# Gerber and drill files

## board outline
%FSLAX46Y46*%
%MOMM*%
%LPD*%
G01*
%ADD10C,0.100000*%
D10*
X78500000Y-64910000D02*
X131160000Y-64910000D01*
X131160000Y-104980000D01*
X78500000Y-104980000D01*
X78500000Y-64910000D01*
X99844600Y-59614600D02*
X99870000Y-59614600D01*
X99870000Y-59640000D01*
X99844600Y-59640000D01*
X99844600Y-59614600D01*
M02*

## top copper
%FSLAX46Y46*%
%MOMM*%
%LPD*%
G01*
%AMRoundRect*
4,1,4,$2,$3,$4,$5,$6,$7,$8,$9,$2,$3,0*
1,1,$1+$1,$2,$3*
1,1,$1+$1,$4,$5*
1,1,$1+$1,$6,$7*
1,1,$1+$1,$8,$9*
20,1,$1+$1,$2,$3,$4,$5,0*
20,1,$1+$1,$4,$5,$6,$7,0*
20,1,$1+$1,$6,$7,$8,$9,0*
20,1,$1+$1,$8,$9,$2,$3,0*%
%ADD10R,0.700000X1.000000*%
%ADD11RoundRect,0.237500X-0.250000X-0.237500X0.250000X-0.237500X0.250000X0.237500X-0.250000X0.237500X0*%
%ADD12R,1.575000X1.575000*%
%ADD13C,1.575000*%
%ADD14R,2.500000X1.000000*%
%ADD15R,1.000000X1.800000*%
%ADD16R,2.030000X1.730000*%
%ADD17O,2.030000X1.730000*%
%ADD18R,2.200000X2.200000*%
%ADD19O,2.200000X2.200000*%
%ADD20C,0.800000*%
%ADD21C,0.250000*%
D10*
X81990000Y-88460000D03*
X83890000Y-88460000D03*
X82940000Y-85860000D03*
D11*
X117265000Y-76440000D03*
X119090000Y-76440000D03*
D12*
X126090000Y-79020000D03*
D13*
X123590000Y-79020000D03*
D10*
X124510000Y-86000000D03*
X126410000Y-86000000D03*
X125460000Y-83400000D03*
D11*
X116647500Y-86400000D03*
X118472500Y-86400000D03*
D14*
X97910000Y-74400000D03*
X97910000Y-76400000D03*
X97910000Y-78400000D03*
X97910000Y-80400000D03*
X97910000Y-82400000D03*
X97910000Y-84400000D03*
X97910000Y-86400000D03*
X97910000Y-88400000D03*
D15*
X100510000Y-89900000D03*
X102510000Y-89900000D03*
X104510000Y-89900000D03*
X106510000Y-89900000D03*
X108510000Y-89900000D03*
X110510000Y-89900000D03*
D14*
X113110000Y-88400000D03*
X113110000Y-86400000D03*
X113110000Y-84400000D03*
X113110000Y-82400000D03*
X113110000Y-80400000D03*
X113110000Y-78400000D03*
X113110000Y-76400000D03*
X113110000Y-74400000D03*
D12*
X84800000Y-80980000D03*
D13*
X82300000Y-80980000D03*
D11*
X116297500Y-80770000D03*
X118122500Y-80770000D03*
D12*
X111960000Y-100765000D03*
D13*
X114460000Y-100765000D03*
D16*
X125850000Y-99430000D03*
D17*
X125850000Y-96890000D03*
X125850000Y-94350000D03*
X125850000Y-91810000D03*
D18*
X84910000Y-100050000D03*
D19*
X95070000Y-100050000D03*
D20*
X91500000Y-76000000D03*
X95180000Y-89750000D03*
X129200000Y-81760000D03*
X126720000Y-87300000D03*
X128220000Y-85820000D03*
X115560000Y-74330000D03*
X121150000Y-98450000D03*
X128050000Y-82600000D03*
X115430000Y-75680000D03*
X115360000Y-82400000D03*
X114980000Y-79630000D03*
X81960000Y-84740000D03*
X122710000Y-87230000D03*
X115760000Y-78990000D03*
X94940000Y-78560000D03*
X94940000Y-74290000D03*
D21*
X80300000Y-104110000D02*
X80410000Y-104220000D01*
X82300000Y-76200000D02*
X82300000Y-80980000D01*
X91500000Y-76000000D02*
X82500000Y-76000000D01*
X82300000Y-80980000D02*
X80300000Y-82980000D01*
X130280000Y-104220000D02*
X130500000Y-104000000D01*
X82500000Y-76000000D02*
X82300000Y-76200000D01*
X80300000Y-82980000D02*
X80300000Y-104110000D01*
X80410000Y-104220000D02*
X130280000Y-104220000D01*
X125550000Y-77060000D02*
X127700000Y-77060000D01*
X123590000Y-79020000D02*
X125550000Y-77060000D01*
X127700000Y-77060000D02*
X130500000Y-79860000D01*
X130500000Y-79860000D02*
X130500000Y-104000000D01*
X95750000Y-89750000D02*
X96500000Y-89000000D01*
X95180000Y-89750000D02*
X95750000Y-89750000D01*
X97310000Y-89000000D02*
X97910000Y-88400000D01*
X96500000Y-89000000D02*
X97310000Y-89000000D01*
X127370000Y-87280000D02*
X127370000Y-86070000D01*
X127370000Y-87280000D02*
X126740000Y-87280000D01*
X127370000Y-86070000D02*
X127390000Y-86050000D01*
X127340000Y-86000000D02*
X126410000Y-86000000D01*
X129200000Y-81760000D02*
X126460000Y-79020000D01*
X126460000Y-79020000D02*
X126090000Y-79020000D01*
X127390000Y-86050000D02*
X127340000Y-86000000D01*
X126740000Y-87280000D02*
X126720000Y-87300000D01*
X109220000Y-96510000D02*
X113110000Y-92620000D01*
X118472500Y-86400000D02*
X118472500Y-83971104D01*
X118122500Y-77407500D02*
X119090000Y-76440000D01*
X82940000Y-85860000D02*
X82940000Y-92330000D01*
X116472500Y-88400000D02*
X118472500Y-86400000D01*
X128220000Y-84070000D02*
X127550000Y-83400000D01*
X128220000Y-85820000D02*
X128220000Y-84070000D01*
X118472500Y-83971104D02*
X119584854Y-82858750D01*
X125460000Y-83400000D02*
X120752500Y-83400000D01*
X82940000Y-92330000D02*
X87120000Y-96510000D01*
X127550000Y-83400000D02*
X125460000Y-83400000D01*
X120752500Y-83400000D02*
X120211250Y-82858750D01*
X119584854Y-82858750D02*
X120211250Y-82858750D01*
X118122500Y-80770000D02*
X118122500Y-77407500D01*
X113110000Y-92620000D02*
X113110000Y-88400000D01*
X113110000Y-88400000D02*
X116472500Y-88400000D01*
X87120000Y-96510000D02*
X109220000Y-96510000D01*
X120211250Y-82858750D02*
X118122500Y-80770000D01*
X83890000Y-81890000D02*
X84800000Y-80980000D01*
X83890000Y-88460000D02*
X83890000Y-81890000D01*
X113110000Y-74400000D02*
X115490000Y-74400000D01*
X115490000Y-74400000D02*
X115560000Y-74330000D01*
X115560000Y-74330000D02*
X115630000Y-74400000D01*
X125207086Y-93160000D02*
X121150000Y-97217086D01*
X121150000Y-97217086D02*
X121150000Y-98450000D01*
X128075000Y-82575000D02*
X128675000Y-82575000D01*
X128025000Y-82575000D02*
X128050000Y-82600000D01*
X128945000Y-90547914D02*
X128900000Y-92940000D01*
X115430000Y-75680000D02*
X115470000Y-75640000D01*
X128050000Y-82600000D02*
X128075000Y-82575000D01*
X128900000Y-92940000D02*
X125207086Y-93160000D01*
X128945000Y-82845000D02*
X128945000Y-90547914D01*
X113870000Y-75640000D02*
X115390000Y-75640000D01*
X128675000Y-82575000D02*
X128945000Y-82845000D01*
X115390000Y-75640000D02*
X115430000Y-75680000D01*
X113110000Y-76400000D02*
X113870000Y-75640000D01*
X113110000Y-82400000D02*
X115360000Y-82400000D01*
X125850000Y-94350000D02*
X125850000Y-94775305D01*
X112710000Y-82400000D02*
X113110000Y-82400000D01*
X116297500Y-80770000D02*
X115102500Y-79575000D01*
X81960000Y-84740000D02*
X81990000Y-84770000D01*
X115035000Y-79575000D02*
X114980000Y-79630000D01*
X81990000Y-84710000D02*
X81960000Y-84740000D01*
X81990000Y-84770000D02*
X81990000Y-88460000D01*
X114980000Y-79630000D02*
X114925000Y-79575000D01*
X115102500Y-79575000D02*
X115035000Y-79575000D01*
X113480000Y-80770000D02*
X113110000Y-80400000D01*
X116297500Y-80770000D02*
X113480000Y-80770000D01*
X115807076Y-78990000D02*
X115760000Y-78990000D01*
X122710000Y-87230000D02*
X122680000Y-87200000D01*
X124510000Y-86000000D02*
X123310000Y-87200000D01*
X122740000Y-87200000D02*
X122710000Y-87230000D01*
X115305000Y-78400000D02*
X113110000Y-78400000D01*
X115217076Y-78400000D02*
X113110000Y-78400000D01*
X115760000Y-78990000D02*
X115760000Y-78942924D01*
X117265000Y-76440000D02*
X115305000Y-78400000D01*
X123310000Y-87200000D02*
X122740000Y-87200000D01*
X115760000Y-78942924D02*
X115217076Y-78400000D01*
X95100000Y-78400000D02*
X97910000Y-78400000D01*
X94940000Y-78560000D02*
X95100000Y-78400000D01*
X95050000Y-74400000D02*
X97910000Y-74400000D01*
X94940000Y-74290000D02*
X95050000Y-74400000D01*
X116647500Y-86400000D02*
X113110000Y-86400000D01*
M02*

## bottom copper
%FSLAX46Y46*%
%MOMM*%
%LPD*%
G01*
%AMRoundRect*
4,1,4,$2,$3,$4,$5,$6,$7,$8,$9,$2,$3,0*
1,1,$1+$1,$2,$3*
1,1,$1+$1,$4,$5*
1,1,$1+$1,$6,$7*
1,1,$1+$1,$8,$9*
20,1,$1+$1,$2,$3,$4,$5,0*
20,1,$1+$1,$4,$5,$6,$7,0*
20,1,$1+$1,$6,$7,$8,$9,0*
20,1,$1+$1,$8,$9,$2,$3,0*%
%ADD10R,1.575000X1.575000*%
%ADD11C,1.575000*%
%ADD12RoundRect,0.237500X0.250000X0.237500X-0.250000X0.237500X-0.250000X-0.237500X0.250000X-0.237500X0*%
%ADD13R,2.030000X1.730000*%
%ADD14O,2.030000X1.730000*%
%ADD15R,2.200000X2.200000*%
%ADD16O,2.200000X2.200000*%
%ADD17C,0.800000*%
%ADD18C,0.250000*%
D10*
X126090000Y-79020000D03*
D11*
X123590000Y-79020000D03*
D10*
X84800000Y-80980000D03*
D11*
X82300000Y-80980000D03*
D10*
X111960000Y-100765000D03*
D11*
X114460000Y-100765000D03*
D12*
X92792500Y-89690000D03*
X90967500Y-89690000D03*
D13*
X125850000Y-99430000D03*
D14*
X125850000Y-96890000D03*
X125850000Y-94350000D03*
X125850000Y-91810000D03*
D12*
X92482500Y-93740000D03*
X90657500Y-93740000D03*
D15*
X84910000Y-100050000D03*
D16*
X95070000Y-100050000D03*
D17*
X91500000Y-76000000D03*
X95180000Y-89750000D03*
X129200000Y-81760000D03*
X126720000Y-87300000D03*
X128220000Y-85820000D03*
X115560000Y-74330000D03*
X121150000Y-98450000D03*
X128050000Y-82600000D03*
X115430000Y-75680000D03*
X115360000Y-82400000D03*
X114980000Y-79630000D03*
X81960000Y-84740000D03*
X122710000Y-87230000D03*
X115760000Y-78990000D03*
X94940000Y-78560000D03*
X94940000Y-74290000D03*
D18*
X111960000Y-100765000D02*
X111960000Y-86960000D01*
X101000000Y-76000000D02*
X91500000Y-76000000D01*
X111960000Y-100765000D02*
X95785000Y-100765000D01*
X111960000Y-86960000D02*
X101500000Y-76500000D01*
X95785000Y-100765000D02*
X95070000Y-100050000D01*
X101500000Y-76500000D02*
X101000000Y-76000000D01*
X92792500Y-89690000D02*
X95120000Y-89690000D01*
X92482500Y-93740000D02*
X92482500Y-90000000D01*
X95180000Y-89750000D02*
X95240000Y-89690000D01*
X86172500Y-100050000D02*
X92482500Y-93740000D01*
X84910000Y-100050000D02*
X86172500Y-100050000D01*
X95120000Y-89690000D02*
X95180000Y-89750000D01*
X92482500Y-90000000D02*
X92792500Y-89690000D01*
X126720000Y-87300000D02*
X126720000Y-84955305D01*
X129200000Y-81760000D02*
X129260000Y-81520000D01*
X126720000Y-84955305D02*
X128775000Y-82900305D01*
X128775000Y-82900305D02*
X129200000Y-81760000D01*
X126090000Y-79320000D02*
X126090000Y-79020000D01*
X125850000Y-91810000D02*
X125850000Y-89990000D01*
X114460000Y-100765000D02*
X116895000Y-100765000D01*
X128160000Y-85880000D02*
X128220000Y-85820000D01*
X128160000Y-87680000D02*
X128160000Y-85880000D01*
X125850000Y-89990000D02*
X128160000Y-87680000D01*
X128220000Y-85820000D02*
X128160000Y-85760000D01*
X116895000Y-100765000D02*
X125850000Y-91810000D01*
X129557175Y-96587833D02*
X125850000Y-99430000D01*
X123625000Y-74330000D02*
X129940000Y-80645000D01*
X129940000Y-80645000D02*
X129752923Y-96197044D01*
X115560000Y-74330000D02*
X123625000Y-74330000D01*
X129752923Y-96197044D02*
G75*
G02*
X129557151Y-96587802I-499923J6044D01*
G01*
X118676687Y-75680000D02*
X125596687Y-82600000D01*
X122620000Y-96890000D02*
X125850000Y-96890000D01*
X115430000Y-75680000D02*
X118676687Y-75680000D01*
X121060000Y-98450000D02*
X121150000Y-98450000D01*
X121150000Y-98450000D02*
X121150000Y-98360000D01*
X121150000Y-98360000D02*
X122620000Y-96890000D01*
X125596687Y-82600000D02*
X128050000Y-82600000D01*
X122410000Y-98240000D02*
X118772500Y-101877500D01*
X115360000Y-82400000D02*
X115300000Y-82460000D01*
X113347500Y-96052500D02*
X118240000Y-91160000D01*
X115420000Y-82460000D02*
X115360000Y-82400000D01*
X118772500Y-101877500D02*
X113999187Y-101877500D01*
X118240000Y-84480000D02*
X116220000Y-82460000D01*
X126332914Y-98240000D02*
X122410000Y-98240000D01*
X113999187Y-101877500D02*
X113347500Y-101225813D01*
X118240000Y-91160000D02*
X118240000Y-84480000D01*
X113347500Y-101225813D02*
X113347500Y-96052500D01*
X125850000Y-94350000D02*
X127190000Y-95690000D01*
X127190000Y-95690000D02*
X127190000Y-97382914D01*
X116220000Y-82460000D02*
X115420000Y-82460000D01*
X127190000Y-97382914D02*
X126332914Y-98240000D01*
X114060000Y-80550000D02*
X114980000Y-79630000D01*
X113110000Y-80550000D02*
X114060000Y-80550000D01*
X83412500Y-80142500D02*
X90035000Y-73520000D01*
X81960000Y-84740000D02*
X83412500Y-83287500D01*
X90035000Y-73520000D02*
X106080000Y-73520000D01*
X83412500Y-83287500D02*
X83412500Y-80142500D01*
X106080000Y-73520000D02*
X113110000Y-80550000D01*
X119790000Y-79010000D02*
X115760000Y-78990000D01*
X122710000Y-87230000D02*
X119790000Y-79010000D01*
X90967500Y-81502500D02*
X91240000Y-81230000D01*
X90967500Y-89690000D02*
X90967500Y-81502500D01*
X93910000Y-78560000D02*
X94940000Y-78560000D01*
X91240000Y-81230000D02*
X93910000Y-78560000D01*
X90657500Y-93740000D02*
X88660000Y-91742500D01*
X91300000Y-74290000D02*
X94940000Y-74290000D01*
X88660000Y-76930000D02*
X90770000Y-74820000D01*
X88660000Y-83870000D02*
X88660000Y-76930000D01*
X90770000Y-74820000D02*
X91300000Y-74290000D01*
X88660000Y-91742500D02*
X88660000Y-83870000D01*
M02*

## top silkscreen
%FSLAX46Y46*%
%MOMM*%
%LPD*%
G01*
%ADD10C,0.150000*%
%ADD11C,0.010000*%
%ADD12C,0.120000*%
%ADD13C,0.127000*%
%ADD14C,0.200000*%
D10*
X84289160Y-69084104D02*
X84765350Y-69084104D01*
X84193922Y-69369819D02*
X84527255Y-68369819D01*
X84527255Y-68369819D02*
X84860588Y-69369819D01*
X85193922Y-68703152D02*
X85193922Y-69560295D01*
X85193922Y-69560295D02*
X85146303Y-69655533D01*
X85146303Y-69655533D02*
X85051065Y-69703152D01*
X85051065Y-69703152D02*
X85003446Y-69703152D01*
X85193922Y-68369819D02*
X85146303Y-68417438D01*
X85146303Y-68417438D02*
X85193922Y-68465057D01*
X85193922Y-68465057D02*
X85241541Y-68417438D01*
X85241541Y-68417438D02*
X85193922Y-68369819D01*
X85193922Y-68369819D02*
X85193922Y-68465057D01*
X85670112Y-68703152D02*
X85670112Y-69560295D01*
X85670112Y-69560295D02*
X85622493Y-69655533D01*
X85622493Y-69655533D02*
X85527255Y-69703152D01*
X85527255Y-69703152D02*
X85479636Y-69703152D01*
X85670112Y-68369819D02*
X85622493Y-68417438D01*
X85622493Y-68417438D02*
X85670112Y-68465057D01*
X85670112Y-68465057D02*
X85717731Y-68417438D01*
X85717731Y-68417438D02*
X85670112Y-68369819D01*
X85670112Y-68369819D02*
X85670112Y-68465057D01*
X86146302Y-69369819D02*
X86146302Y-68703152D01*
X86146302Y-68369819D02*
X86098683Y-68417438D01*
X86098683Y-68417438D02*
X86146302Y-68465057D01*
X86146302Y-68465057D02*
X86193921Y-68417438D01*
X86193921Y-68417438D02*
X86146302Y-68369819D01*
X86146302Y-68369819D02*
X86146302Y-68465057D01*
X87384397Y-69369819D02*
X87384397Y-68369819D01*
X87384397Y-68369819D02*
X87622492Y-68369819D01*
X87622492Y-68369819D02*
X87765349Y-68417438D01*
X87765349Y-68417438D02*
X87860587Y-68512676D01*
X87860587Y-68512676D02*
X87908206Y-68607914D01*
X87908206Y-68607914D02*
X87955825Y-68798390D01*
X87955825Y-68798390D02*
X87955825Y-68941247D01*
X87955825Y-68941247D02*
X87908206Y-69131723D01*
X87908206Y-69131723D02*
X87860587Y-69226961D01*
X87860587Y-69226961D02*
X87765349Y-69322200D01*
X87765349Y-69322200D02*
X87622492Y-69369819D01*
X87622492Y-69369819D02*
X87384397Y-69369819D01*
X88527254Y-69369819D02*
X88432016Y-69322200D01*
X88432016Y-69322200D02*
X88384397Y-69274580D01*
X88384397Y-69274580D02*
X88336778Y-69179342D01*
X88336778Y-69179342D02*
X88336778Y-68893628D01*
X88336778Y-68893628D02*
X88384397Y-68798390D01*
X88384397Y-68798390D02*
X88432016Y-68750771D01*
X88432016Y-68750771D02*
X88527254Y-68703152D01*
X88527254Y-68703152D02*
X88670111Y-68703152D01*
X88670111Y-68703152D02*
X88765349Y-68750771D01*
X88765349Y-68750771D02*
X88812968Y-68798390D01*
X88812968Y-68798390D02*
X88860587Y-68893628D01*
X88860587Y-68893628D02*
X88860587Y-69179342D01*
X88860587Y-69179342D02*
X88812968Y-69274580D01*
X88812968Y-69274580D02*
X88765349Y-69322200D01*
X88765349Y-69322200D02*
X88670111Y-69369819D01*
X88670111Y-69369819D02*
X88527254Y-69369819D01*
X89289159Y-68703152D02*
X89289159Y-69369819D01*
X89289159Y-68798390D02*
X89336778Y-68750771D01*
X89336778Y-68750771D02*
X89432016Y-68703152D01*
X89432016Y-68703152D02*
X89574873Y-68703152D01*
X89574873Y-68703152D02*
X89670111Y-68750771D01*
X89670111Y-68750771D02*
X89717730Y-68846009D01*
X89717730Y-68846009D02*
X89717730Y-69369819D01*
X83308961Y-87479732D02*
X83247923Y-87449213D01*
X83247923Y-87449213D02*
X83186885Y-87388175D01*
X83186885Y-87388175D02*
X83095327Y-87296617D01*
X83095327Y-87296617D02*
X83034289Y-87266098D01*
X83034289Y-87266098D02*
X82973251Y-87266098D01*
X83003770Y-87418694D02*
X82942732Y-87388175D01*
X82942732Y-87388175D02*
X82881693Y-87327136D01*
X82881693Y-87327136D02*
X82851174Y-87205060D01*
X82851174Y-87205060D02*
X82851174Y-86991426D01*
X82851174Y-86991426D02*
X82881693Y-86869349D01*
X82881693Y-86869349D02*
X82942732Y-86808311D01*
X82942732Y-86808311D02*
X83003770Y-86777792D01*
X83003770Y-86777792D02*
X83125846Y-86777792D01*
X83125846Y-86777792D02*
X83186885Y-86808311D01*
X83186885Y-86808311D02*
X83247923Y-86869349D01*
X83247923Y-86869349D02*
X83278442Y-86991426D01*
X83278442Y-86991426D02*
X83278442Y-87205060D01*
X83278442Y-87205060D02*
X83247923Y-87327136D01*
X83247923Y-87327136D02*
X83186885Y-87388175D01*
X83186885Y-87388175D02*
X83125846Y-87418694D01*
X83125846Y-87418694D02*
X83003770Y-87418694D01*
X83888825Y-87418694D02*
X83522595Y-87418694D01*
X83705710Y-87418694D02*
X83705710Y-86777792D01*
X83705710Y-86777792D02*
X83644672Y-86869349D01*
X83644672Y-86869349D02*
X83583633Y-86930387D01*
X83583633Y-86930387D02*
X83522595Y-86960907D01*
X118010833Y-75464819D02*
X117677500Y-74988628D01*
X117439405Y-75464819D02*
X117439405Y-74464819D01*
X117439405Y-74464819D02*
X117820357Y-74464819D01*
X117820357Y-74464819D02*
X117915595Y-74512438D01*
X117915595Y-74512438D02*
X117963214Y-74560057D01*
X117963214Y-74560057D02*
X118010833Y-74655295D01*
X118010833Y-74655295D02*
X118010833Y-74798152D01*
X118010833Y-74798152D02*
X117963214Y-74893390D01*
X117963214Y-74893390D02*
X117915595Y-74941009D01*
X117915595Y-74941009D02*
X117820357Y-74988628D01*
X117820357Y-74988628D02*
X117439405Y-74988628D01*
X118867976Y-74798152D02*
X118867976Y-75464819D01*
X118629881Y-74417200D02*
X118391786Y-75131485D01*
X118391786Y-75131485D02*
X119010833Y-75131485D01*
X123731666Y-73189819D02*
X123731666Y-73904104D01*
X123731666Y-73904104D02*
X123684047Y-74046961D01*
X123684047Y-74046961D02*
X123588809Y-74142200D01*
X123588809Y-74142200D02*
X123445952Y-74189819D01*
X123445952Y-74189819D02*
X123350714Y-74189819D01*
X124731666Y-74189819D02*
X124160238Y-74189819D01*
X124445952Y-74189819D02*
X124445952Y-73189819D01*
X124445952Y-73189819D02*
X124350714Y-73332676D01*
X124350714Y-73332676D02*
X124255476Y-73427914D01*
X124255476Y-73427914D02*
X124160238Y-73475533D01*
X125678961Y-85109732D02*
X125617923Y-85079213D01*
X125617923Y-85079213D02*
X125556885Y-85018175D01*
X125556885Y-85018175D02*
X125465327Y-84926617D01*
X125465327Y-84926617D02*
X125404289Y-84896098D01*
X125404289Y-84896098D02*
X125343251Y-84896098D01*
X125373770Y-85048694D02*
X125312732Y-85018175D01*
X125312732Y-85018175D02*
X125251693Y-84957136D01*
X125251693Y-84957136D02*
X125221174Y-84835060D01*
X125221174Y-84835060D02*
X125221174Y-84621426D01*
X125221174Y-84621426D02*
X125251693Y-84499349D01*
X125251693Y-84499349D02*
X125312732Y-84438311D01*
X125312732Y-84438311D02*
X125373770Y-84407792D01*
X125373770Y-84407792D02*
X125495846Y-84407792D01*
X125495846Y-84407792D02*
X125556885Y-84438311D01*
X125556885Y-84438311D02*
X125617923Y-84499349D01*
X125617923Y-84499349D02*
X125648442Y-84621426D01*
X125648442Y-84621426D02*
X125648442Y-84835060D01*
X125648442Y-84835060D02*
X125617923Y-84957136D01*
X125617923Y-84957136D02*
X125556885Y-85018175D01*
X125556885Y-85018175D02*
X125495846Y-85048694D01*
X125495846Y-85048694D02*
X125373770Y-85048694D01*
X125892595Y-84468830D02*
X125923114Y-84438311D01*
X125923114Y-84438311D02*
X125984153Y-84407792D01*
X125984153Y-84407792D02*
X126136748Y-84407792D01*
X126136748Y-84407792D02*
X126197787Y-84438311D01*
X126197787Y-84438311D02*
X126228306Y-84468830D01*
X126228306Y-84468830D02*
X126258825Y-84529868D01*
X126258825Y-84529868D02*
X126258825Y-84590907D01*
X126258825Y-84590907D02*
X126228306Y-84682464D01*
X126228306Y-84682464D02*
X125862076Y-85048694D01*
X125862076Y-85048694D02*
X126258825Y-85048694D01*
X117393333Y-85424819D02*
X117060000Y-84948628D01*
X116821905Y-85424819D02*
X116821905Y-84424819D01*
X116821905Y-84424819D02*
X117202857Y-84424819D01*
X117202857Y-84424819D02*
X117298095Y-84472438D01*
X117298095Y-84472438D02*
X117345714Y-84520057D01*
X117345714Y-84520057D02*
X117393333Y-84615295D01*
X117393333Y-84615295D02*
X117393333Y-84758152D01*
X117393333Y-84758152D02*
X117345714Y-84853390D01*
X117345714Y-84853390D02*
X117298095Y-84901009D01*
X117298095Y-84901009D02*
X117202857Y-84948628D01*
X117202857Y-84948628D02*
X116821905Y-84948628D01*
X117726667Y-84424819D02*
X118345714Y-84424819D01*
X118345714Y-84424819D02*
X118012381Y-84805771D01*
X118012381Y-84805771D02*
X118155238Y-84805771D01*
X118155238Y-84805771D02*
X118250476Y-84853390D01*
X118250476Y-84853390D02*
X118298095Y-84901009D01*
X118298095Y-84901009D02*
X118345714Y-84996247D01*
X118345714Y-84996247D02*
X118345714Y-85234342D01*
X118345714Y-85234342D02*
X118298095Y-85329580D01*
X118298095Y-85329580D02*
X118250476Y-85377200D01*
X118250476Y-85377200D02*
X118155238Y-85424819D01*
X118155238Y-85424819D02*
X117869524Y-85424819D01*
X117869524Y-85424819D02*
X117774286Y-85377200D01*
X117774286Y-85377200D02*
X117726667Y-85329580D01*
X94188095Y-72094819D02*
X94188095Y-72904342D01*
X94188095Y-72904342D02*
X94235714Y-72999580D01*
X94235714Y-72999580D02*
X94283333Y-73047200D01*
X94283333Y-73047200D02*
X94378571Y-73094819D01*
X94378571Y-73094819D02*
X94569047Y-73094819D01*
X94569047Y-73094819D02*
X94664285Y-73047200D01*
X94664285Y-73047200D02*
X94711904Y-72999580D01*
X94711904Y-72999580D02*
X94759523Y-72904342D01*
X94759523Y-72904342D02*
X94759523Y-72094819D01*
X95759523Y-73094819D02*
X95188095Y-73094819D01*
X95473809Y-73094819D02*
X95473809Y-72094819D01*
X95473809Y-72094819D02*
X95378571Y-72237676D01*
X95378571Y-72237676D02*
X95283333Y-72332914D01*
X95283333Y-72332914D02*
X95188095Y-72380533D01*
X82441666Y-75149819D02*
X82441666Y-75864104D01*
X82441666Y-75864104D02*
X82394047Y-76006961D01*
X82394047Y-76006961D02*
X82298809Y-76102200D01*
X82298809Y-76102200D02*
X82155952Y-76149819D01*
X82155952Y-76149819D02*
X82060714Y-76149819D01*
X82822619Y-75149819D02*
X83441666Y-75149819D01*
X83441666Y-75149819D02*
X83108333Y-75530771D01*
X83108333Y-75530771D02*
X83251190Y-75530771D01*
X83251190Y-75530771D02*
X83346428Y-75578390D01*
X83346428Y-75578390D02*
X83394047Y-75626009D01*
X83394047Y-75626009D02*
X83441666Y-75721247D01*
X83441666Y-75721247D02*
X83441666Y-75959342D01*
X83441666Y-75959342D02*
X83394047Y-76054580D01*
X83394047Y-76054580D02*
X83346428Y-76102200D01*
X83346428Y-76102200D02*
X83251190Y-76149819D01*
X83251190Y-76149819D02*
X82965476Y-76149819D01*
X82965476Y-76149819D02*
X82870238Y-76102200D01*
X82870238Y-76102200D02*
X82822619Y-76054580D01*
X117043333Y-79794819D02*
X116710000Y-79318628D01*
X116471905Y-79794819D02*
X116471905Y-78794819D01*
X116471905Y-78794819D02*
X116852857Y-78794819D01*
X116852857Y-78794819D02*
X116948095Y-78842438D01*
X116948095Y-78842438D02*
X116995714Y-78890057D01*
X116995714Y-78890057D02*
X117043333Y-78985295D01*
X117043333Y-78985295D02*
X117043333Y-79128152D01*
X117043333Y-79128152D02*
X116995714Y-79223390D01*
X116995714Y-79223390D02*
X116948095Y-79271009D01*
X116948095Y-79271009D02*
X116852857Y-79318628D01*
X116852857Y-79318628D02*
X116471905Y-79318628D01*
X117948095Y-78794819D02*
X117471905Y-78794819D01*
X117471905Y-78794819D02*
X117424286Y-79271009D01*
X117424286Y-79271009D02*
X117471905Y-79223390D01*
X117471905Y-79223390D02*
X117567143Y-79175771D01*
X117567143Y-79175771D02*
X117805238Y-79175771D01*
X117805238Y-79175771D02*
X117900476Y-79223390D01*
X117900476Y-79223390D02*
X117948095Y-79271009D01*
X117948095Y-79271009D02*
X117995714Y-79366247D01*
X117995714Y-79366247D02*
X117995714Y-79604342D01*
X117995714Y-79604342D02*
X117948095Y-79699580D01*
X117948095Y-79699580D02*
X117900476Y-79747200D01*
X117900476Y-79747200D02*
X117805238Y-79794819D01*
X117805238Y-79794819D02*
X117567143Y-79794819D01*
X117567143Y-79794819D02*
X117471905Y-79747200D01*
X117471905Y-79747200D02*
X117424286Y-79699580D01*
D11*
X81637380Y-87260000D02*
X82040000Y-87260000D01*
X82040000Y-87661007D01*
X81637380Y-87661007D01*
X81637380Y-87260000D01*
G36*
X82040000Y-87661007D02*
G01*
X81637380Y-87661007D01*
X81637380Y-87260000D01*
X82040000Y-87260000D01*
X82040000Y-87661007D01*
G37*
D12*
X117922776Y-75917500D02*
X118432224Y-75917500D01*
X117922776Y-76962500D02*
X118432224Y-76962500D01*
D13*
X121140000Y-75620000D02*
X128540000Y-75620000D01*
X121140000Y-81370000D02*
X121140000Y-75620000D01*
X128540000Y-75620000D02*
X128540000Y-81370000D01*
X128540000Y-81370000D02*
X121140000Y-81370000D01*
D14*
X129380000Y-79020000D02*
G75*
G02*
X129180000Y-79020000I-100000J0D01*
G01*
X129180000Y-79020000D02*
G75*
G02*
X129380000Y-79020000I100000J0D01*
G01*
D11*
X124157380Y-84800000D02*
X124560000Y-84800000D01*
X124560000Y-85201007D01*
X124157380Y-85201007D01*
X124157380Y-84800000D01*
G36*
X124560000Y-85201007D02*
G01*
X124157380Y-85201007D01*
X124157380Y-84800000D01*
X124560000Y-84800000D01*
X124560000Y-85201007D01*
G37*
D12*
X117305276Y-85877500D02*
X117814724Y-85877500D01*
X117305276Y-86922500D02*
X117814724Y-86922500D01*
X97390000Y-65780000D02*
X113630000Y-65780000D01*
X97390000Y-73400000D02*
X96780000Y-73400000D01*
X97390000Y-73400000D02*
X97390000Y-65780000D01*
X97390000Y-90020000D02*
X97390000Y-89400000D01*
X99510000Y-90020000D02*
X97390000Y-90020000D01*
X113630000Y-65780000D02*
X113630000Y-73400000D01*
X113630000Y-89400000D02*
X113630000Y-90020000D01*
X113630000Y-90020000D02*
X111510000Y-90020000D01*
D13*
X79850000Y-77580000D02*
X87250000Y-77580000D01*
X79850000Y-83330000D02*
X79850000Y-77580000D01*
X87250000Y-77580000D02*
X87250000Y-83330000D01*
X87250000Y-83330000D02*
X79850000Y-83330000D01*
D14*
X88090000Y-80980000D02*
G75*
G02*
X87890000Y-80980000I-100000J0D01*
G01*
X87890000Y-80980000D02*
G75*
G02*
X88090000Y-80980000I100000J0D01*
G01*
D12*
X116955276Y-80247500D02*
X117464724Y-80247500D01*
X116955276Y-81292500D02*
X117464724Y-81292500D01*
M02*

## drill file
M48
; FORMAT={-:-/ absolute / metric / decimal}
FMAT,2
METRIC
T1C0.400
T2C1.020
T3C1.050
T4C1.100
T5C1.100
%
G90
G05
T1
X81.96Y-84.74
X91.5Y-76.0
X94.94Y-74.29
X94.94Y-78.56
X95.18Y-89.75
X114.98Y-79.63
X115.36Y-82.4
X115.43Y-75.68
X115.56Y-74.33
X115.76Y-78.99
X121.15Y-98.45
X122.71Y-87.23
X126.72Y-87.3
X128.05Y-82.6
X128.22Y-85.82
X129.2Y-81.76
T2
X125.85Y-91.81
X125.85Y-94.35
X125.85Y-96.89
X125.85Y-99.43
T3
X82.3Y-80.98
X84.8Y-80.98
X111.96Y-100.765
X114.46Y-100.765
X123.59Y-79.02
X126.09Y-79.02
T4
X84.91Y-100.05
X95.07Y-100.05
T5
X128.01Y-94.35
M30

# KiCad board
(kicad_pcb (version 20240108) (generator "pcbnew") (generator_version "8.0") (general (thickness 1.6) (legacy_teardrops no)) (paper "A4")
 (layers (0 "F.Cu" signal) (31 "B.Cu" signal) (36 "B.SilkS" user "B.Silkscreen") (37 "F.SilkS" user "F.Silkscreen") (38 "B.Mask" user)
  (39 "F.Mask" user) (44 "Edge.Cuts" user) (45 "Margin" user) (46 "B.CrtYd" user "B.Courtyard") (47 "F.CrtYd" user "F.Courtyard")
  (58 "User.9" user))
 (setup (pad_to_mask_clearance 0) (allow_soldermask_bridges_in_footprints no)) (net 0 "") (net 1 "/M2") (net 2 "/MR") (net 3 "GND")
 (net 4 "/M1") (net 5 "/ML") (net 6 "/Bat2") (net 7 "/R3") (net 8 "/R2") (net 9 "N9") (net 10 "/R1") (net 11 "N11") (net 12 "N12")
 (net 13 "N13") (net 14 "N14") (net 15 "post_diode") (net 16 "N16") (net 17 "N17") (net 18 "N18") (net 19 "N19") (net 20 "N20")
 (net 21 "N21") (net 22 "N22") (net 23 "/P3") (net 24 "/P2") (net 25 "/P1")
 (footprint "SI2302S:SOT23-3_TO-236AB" (layer "F.Cu") (at 82.94 87.16)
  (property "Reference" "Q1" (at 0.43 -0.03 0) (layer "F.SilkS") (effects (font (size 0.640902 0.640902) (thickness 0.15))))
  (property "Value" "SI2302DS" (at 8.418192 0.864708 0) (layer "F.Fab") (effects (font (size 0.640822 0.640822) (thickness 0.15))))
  (fp_poly
   (pts (xy -1.30262 0.1) (xy -0.9 0.1) (xy -0.9 0.501007) (xy -1.30262 0.501007)) (stroke (width 0.01) (type solid)) (fill solid)
   (layer "F.SilkS"))
  (pad "1" smd rect (at -0.95 1.3) (size 0.7 1) (layers "F.Cu" "F.Paste" "F.Mask") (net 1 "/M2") (solder_mask_margin 0.102))
  (pad "2" smd rect (at 0.95 1.3) (size 0.7 1) (layers "F.Cu" "F.Paste" "F.Mask") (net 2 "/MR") (solder_mask_margin 0.102))
  (pad "3" smd rect (at 0 -1.3) (size 0.7 1) (layers "F.Cu" "F.Paste" "F.Mask") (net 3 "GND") (solder_mask_margin 0.102)))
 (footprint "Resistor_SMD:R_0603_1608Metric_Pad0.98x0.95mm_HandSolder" (layer "F.Cu") (at 118.1775 76.44)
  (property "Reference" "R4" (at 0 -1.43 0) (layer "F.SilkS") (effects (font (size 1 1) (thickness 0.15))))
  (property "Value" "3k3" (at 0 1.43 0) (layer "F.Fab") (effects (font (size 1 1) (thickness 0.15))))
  (fp_line (start -0.254724 -0.5225) (end 0.254724 -0.5225) (stroke (width 0.12) (type solid)) (layer "F.SilkS"))
  (fp_line (start -0.254724 0.5225) (end 0.254724 0.5225) (stroke (width 0.12) (type solid)) (layer "F.SilkS"))
  (pad "1" smd roundrect (at -0.9125 0) (size 0.975 0.95) (layers "F.Cu" "F.Paste" "F.Mask") (roundrect_rratio 0.25) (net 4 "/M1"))
  (pad "2" smd roundrect (at 0.9125 0) (size 0.975 0.95) (layers "F.Cu" "F.Paste" "F.Mask") (roundrect_rratio 0.25) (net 3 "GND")))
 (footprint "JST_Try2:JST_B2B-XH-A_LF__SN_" (layer "F.Cu") (at 124.84 78.495)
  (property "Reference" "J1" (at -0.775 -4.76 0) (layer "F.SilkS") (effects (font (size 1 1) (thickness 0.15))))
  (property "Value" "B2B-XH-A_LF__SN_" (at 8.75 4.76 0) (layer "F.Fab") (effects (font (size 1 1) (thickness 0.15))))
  (fp_line (start -3.7 -2.875) (end 3.7 -2.875) (stroke (width 0.127) (type solid)) (layer "F.SilkS"))
  (fp_line (start -3.7 2.875) (end -3.7 -2.875) (stroke (width 0.127) (type solid)) (layer "F.SilkS"))
  (fp_line (start 3.7 -2.875) (end 3.7 2.875) (stroke (width 0.127) (type solid)) (layer "F.SilkS"))
  (fp_line (start 3.7 2.875) (end -3.7 2.875) (stroke (width 0.127) (type solid)) (layer "F.SilkS"))
  (fp_circle (center 4.44 0.525) (end 4.54 0.525) (stroke (width 0.2) (type solid)) (fill none) (layer "F.SilkS"))
  (pad "1" thru_hole rect (at 1.25 0.525) (size 1.575 1.575) (drill 1.05) (layers "*.Cu" "*.Mask") (remove_unused_layers no) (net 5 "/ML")
   (solder_mask_margin 0.102))
  (pad "2" thru_hole circle (at -1.25 0.525) (size 1.575 1.575) (drill 1.05) (layers "*.Cu" "*.Mask") (remove_unused_layers no)
   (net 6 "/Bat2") (solder_mask_margin 0.102)))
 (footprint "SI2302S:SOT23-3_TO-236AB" (layer "F.Cu") (at 125.46 84.7)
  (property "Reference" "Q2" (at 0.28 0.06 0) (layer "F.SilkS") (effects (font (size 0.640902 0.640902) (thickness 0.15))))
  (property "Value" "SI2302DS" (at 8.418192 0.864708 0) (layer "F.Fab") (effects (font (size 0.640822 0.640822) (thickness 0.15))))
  (fp_poly
   (pts (xy -1.30262 0.1) (xy -0.9 0.1) (xy -0.9 0.501007) (xy -1.30262 0.501007)) (stroke (width 0.01) (type solid)) (fill solid)
   (layer "F.SilkS"))
  (pad "1" smd rect (at -0.95 1.3) (size 0.7 1) (layers "F.Cu" "F.Paste" "F.Mask") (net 4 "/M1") (solder_mask_margin 0.102))
  (pad "2" smd rect (at 0.95 1.3) (size 0.7 1) (layers "F.Cu" "F.Paste" "F.Mask") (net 5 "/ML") (solder_mask_margin 0.102))
  (pad "3" smd rect (at 0 -1.3) (size 0.7 1) (layers "F.Cu" "F.Paste" "F.Mask") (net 3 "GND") (solder_mask_margin 0.102)))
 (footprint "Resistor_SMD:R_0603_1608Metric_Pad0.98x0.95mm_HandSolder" (layer "F.Cu") (at 117.56 86.4)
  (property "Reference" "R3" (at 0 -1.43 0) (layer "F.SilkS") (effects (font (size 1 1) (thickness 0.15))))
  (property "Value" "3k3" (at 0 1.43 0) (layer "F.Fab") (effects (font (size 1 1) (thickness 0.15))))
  (fp_line (start -0.254724 -0.5225) (end 0.254724 -0.5225) (stroke (width 0.12) (type solid)) (layer "F.SilkS"))
  (fp_line (start -0.254724 0.5225) (end 0.254724 0.5225) (stroke (width 0.12) (type solid)) (layer "F.SilkS"))
  (pad "1" smd roundrect (at -0.9125 0) (size 0.975 0.95) (layers "F.Cu" "F.Paste" "F.Mask") (roundrect_rratio 0.25) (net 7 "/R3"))
  (pad "2" smd roundrect (at 0.9125 0) (size 0.975 0.95) (layers "F.Cu" "F.Paste" "F.Mask") (roundrect_rratio 0.25) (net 3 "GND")))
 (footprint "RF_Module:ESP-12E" (layer "F.Cu") (at 105.51 77.9)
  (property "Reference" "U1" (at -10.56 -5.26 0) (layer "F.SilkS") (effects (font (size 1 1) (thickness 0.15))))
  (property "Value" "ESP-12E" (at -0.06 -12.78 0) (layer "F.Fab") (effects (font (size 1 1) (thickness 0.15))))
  (fp_line (start -8.12 -12.12) (end 8.12 -12.12) (stroke (width 0.12) (type solid)) (layer "F.SilkS"))
  (fp_line (start -8.12 -4.5) (end -8.73 -4.5) (stroke (width 0.12) (type solid)) (layer "F.SilkS"))
  (fp_line (start -8.12 -4.5) (end -8.12 -12.12) (stroke (width 0.12) (type solid)) (layer "F.SilkS"))
  (fp_line (start -8.12 12.12) (end -8.12 11.5) (stroke (width 0.12) (type solid)) (layer "F.SilkS"))
  (fp_line (start -6 12.12) (end -8.12 12.12) (stroke (width 0.12) (type solid)) (layer "F.SilkS"))
  (fp_line (start 8.12 -12.12) (end 8.12 -4.5) (stroke (width 0.12) (type solid)) (layer "F.SilkS"))
  (fp_line (start 8.12 11.5) (end 8.12 12.12) (stroke (width 0.12) (type solid)) (layer "F.SilkS"))
  (fp_line (start 8.12 12.12) (end 6 12.12) (stroke (width 0.12) (type solid)) (layer "F.SilkS"))
  (pad "1" smd rect (at -7.6 -3.5) (size 2.5 1) (layers "F.Cu" "F.Mask") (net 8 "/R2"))
  (pad "2" smd rect (at -7.6 -1.5) (size 2.5 1) (layers "F.Cu" "F.Mask") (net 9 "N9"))
  (pad "3" smd rect (at -7.6 0.5) (size 2.5 1) (layers "F.Cu" "F.Mask") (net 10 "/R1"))
  (pad "4" smd rect (at -7.6 2.5) (size 2.5 1) (layers "F.Cu" "F.Mask") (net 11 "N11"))
  (pad "5" smd rect (at -7.6 4.5) (size 2.5 1) (layers "F.Cu" "F.Mask") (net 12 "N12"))
  (pad "6" smd rect (at -7.6 6.5) (size 2.5 1) (layers "F.Cu" "F.Mask") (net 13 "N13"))
  (pad "7" smd rect (at -7.6 8.5) (size 2.5 1) (layers "F.Cu" "F.Mask") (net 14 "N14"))
  (pad "8" smd rect (at -7.6 10.5) (size 2.5 1) (layers "F.Cu" "F.Mask") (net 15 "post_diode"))
  (pad "9" smd rect (at -5 12) (size 1 1.8) (layers "F.Cu" "F.Mask") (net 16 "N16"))
  (pad "10" smd rect (at -3 12) (size 1 1.8) (layers "F.Cu" "F.Mask") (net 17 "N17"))
  (pad "11" smd rect (at -1 12) (size 1 1.8) (layers "F.Cu" "F.Mask") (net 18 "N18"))
  (pad "12" smd rect (at 1 12) (size 1 1.8) (layers "F.Cu" "F.Mask") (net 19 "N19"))
  (pad "13" smd rect (at 3 12) (size 1 1.8) (layers "F.Cu" "F.Mask") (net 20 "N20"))
  (pad "14" smd rect (at 5 12) (size 1 1.8) (layers "F.Cu" "F.Mask") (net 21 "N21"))
  (pad "15" smd rect (at 7.6 10.5) (size 2.5 1) (layers "F.Cu" "F.Mask") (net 3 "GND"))
  (pad "16" smd rect (at 7.6 8.5) (size 2.5 1) (layers "F.Cu" "F.Mask") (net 7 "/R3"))
  (pad "17" smd rect (at 7.6 6.5) (size 2.5 1) (layers "F.Cu" "F.Mask") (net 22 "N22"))
  (pad "18" smd rect (at 7.6 4.5) (size 2.5 1) (layers "F.Cu" "F.Mask") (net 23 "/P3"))
  (pad "19" smd rect (at 7.6 2.5) (size 2.5 1) (layers "F.Cu" "F.Mask") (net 1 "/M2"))
  (pad "20" smd rect (at 7.6 0.5) (size 2.5 1) (layers "F.Cu" "F.Mask") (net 4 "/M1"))
  (pad "21" smd rect (at 7.6 -1.5) (size 2.5 1) (layers "F.Cu" "F.Mask") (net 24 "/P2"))
  (pad "22" smd rect (at 7.6 -3.5) (size 2.5 1) (layers "F.Cu" "F.Mask") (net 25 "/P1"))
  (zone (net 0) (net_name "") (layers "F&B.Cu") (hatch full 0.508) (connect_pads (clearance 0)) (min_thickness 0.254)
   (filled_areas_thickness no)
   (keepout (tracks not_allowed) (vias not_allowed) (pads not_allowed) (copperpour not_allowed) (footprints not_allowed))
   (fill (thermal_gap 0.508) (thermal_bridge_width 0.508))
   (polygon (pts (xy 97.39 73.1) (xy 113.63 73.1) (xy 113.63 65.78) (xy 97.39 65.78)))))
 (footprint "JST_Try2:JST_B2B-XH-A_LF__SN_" (layer "F.Cu") (at 83.55 80.455)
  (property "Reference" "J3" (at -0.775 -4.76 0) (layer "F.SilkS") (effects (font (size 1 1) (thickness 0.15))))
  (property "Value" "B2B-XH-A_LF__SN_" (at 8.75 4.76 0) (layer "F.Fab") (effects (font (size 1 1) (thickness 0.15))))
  (fp_line (start -3.7 -2.875) (end 3.7 -2.875) (stroke (width 0.127) (type solid)) (layer "F.SilkS"))
  (fp_line (start -3.7 2.875) (end -3.7 -2.875) (stroke (width 0.127) (type solid)) (layer "F.SilkS"))
  (fp_line (start 3.7 -2.875) (end 3.7 2.875) (stroke (width 0.127) (type solid)) (layer "F.SilkS"))
  (fp_line (start 3.7 2.875) (end -3.7 2.875) (stroke (width 0.127) (type solid)) (layer "F.SilkS"))
  (fp_circle (center 4.44 0.525) (end 4.54 0.525) (stroke (width 0.2) (type solid)) (fill none) (layer "F.SilkS"))
  (pad "1" thru_hole rect (at 1.25 0.525) (size 1.575 1.575) (drill 1.05) (layers "*.Cu" "*.Mask") (remove_unused_layers no) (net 2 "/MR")
   (solder_mask_margin 0.102))
  (pad "2" thru_hole circle (at -1.25 0.525) (size 1.575 1.575) (drill 1.05) (layers "*.Cu" "*.Mask") (remove_unused_layers no)
   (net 6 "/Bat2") (solder_mask_margin 0.102)))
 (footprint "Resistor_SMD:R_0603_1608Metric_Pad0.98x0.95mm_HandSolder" (layer "F.Cu") (at 117.21 80.77)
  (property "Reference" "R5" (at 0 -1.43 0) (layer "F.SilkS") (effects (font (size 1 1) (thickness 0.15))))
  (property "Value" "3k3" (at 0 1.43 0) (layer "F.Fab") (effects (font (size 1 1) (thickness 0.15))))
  (fp_line (start -0.254724 -0.5225) (end 0.254724 -0.5225) (stroke (width 0.12) (type solid)) (layer "F.SilkS"))
  (fp_line (start -0.254724 0.5225) (end 0.254724 0.5225) (stroke (width 0.12) (type solid)) (layer "F.SilkS"))
  (pad "1" smd roundrect (at -0.9125 0) (size 0.975 0.95) (layers "F.Cu" "F.Paste" "F.Mask") (roundrect_rratio 0.25) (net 1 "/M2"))
  (pad "2" smd roundrect (at 0.9125 0) (size 0.975 0.95) (layers "F.Cu" "F.Paste" "F.Mask") (roundrect_rratio 0.25) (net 3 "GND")))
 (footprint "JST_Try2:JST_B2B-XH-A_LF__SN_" (layer "B.Cu") (at 113.21 100.24 180)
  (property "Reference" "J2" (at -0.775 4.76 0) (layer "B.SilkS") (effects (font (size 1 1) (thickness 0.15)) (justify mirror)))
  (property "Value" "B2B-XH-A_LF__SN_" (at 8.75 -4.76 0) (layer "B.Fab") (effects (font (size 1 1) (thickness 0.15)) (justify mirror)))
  (pad "1" thru_hole rect (at 1.25 -0.525 180) (size 1.575 1.575) (drill 1.05) (layers "*.Cu" "*.Mask") (remove_unused_layers no)
   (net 6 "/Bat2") (solder_mask_margin 0.102))
  (pad "2" thru_hole circle (at -1.25 -0.525 180) (size 1.575 1.575) (drill 1.05) (layers "*.Cu" "*.Mask") (remove_unused_layers no)
   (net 3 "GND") (solder_mask_margin 0.102)))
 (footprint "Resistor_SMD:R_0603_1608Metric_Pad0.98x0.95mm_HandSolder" (layer "B.Cu") (at 91.88 89.69 180)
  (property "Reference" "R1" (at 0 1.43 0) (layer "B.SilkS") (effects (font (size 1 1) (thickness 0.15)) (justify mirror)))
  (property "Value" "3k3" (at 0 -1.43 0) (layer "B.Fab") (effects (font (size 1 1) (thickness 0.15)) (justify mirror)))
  (pad "1" smd roundrect (at -0.9125 0 180) (size 0.975 0.95) (layers "B.Cu" "B.Paste" "B.Mask") (roundrect_rratio 0.25)
   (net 15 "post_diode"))
  (pad "2" smd roundrect (at 0.9125 0 180) (size 0.975 0.95) (layers "B.Cu" "B.Paste" "B.Mask") (roundrect_rratio 0.25) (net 10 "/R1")))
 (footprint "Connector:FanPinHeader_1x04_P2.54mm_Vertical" (layer "B.Cu") (at 125.85 99.43 90)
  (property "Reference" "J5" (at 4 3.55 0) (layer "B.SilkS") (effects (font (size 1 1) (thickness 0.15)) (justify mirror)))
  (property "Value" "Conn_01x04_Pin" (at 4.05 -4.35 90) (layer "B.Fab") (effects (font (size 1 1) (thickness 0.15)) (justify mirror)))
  (pad "" np_thru_hole circle (at 5.08 2.16) (size 1.1 1.1) (drill 1.1) (layers "*.Cu" "*.Mask"))
  (pad "1" thru_hole rect (at 0 0) (size 2.03 1.73) (drill 1.02) (layers "*.Cu" "*.Mask") (remove_unused_layers no) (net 25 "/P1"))
  (pad "2" thru_hole oval (at 2.54 0) (size 2.03 1.73) (drill 1.02) (layers "*.Cu" "*.Mask") (remove_unused_layers no) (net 24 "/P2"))
  (pad "3" thru_hole oval (at 5.08 0) (size 2.03 1.73) (drill 1.02) (layers "*.Cu" "*.Mask") (remove_unused_layers no) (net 23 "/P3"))
  (pad "4" thru_hole oval (at 7.62 0) (size 2.03 1.73) (drill 1.02) (layers "*.Cu" "*.Mask") (remove_unused_layers no) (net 3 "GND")))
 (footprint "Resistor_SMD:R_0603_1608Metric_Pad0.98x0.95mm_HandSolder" (layer "B.Cu") (at 91.57 93.74 180)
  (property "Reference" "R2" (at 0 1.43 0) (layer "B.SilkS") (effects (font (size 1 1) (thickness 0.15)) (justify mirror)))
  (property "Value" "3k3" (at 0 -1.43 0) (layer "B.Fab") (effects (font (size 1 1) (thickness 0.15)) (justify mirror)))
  (pad "1" smd roundrect (at -0.9125 0 180) (size 0.975 0.95) (layers "B.Cu" "B.Paste" "B.Mask") (roundrect_rratio 0.25)
   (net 15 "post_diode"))
  (pad "2" smd roundrect (at 0.9125 0 180) (size 0.975 0.95) (layers "B.Cu" "B.Paste" "B.Mask") (roundrect_rratio 0.25) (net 8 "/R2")))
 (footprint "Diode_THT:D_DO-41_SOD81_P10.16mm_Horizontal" (layer "B.Cu") (at 84.91 100.05)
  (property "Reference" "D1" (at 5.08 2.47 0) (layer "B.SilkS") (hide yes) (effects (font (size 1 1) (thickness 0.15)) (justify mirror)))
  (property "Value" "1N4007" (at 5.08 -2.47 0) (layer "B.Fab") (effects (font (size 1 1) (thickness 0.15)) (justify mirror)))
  (pad "1" thru_hole rect (at 0 0) (size 2.2 2.2) (drill 1.1) (layers "*.Cu" "*.Mask") (remove_unused_layers no) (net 15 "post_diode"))
  (pad "2" thru_hole oval (at 10.16 0) (size 2.2 2.2) (drill 1.1) (layers "*.Cu" "*.Mask") (remove_unused_layers no) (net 6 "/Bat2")))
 (gr_rect (start 78.5 64.91) (end 131.16 104.98) (stroke (width 0.1) (type default)) (fill none) (layer "Edge.Cuts"))
 (gr_rect (start 99.8446 59.6146) (end 99.87 59.64) (stroke (width 0.1) (type default)) (fill none) (layer "Edge.Cuts"))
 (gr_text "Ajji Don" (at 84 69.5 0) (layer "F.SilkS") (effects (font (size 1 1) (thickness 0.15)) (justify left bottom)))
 (segment (start 80.3 104.11) (end 80.41 104.22) (width 0.25) (layer "F.Cu") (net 6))
 (segment (start 82.3 76.2) (end 82.3 80.98) (width 0.25) (layer "F.Cu") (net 6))
 (segment (start 91.5 76) (end 82.5 76) (width 0.25) (layer "F.Cu") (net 6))
 (segment (start 82.3 80.98) (end 80.3 82.98) (width 0.25) (layer "F.Cu") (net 6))
 (segment (start 130.28 104.22) (end 130.5 104) (width 0.25) (layer "F.Cu") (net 6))
 (segment (start 82.5 76) (end 82.3 76.2) (width 0.25) (layer "F.Cu") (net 6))
 (segment (start 80.3 82.98) (end 80.3 104.11) (width 0.25) (layer "F.Cu") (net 6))
 (segment (start 80.41 104.22) (end 130.28 104.22) (width 0.25) (layer "F.Cu") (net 6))
 (segment (start 125.55 77.06) (end 127.7 77.06) (width 0.25) (layer "F.Cu") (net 6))
 (segment (start 123.59 79.02) (end 125.55 77.06) (width 0.25) (layer "F.Cu") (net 6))
 (segment (start 127.7 77.06) (end 130.5 79.86) (width 0.25) (layer "F.Cu") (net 6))
 (segment (start 130.5 79.86) (end 130.5 104) (width 0.25) (layer "F.Cu") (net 6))
 (via (at 91.5 76) (size 0.8) (drill 0.4) (layers "F.Cu" "B.Cu") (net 6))
 (segment (start 111.96 100.765) (end 111.96 86.96) (width 0.25) (layer "B.Cu") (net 6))
 (segment (start 101 76) (end 91.5 76) (width 0.25) (layer "B.Cu") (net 6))
 (segment (start 111.96 100.765) (end 95.785 100.765) (width 0.25) (layer "B.Cu") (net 6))
 (segment (start 111.96 86.96) (end 101.5 76.5) (width 0.25) (layer "B.Cu") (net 6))
 (segment (start 95.785 100.765) (end 95.07 100.05) (width 0.25) (layer "B.Cu") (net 6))
 (segment (start 101.5 76.5) (end 101 76) (width 0.25) (layer "B.Cu") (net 6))
 (segment (start 95.75 89.75) (end 96.5 89) (width 0.25) (layer "F.Cu") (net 15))
 (segment (start 95.18 89.75) (end 95.75 89.75) (width 0.25) (layer "F.Cu") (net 15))
 (segment (start 97.31 89) (end 97.91 88.4) (width 0.25) (layer "F.Cu") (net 15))
 (segment (start 96.5 89) (end 97.31 89) (width 0.25) (layer "F.Cu") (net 15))
 (via (at 95.18 89.75) (size 0.8) (drill 0.4) (layers "F.Cu" "B.Cu") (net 15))
 (segment (start 92.7925 89.69) (end 95.12 89.69) (width 0.25) (layer "B.Cu") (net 15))
 (segment (start 92.4825 93.74) (end 92.4825 90) (width 0.25) (layer "B.Cu") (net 15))
 (segment (start 95.18 89.75) (end 95.24 89.69) (width 0.25) (layer "B.Cu") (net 15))
 (segment (start 86.1725 100.05) (end 92.4825 93.74) (width 0.25) (layer "B.Cu") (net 15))
 (segment (start 84.91 100.05) (end 86.1725 100.05) (width 0.25) (layer "B.Cu") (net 15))
 (segment (start 95.12 89.69) (end 95.18 89.75) (width 0.25) (layer "B.Cu") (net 15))
 (segment (start 92.4825 90) (end 92.7925 89.69) (width 0.25) (layer "B.Cu") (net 15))
 (segment (start 127.37 87.28) (end 127.37 86.07) (width 0.25) (layer "F.Cu") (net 5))
 (segment (start 127.37 87.28) (end 126.74 87.28) (width 0.25) (layer "F.Cu") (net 5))
 (segment (start 127.37 86.07) (end 127.39 86.05) (width 0.25) (layer "F.Cu") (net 5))
 (segment (start 127.34 86) (end 126.41 86) (width 0.25) (layer "F.Cu") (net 5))
 (segment (start 129.2 81.76) (end 126.46 79.02) (width 0.25) (layer "F.Cu") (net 5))
 (segment (start 126.46 79.02) (end 126.09 79.02) (width 0.25) (layer "F.Cu") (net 5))
 (segment (start 127.39 86.05) (end 127.34 86) (width 0.25) (layer "F.Cu") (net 5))
 (segment (start 126.74 87.28) (end 126.72 87.3) (width 0.25) (layer "F.Cu") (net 5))
 (via (at 129.2 81.76) (size 0.8) (drill 0.4) (layers "F.Cu" "B.Cu") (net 5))
 (via (at 126.72 87.3) (size 0.8) (drill 0.4) (layers "F.Cu" "B.Cu") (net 5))
 (segment (start 126.72 87.3) (end 126.72 84.955305) (width 0.25) (layer "B.Cu") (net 5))
 (segment (start 129.2 81.76) (end 129.26 81.52) (width 0.25) (layer "B.Cu") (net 5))
 (segment (start 126.72 84.955305) (end 128.775 82.900305) (width 0.25) (layer "B.Cu") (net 5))
 (segment (start 128.775 82.900305) (end 129.2 81.76) (width 0.25) (layer "B.Cu") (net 5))
 (segment (start 126.09 79.32) (end 126.09 79.02) (width 0.25) (layer "B.Cu") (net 5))
 (segment (start 109.22 96.51) (end 113.11 92.62) (width 0.25) (layer "F.Cu") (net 3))
 (segment (start 118.4725 86.4) (end 118.4725 83.971104) (width 0.25) (layer "F.Cu") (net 3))
 (segment (start 118.1225 77.4075) (end 119.09 76.44) (width 0.25) (layer "F.Cu") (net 3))
 (segment (start 82.94 85.86) (end 82.94 92.33) (width 0.25) (layer "F.Cu") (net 3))
 (segment (start 116.4725 88.4) (end 118.4725 86.4) (width 0.25) (layer "F.Cu") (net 3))
 (segment (start 128.22 84.07) (end 127.55 83.4) (width 0.25) (layer "F.Cu") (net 3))
 (segment (start 128.22 85.82) (end 128.22 84.07) (width 0.25) (layer "F.Cu") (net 3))
 (segment (start 118.4725 83.971104) (end 119.584854 82.85875) (width 0.25) (layer "F.Cu") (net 3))
 (segment (start 125.46 83.4) (end 120.7525 83.4) (width 0.25) (layer "F.Cu") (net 3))
 (segment (start 82.94 92.33) (end 87.12 96.51) (width 0.25) (layer "F.Cu") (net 3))
 (segment (start 127.55 83.4) (end 125.46 83.4) (width 0.25) (layer "F.Cu") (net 3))
 (segment (start 120.7525 83.4) (end 120.21125 82.85875) (width 0.25) (layer "F.Cu") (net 3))
 (segment (start 119.584854 82.85875) (end 120.21125 82.85875) (width 0.25) (layer "F.Cu") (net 3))
 (segment (start 118.1225 80.77) (end 118.1225 77.4075) (width 0.25) (layer "F.Cu") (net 3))
 (segment (start 113.11 92.62) (end 113.11 88.4) (width 0.25) (layer "F.Cu") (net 3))
 (segment (start 113.11 88.4) (end 116.4725 88.4) (width 0.25) (layer "F.Cu") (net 3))
 (segment (start 87.12 96.51) (end 109.22 96.51) (width 0.25) (layer "F.Cu") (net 3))
 (segment (start 120.21125 82.85875) (end 118.1225 80.77) (width 0.25) (layer "F.Cu") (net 3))
 (via (at 128.22 85.82) (size 0.8) (drill 0.4) (layers "F.Cu" "B.Cu") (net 3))
 (segment (start 125.85 91.81) (end 125.85 89.99) (width 0.25) (layer "B.Cu") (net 3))
 (segment (start 114.46 100.765) (end 116.895 100.765) (width 0.25) (layer "B.Cu") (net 3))
 (segment (start 128.16 85.88) (end 128.22 85.82) (width 0.25) (layer "B.Cu") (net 3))
 (segment (start 128.16 87.68) (end 128.16 85.88) (width 0.25) (layer "B.Cu") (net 3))
 (segment (start 125.85 89.99) (end 128.16 87.68) (width 0.25) (layer "B.Cu") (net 3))
 (segment (start 128.22 85.82) (end 128.16 85.76) (width 0.25) (layer "B.Cu") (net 3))
 (segment (start 116.895 100.765) (end 125.85 91.81) (width 0.25) (layer "B.Cu") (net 3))
 (segment (start 83.89 81.89) (end 84.8 80.98) (width 0.25) (layer "F.Cu") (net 2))
 (segment (start 83.89 88.46) (end 83.89 81.89) (width 0.25) (layer "F.Cu") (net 2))
 (segment (start 113.11 74.4) (end 115.49 74.4) (width 0.25) (layer "F.Cu") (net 25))
 (segment (start 115.49 74.4) (end 115.56 74.33) (width 0.25) (layer "F.Cu") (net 25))
 (segment (start 115.56 74.33) (end 115.63 74.4) (width 0.25) (layer "F.Cu") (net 25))
 (via (at 115.56 74.33) (size 0.8) (drill 0.4) (layers "F.Cu" "B.Cu") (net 25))
 (segment (start 129.557175 96.587833) (end 125.85 99.43) (width 0.25) (layer "B.Cu") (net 25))
 (segment (start 123.625 74.33) (end 129.94 80.645) (width 0.25) (layer "B.Cu") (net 25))
 (segment (start 129.94 80.645) (end 129.752923 96.197044) (width 0.25) (layer "B.Cu") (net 25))
 (segment (start 115.56 74.33) (end 123.625 74.33) (width 0.25) (layer "B.Cu") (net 25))
 (arc (start 129.752923 96.197044) (mid 129.700011 96.41496) (end 129.557175 96.587833) (width 0.25) (layer "B.Cu") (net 25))
 (segment (start 125.207086 93.16) (end 121.15 97.217086) (width 0.25) (layer "F.Cu") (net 24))
 (segment (start 121.15 97.217086) (end 121.15 98.45) (width 0.25) (layer "F.Cu") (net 24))
 (segment (start 128.075 82.575) (end 128.675 82.575) (width 0.25) (layer "F.Cu") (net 24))
 (segment (start 128.025 82.575) (end 128.05 82.6) (width 0.25) (layer "F.Cu") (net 24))
 (segment (start 128.945 90.547914) (end 128.9 92.94) (width 0.25) (layer "F.Cu") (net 24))
 (segment (start 115.43 75.68) (end 115.47 75.64) (width 0.25) (layer "F.Cu") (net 24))
 (segment (start 128.05 82.6) (end 128.075 82.575) (width 0.25) (layer "F.Cu") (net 24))
 (segment (start 128.9 92.94) (end 125.207086 93.16) (width 0.25) (layer "F.Cu") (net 24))
 (segment (start 128.945 82.845) (end 128.945 90.547914) (width 0.25) (layer "F.Cu") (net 24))
 (segment (start 113.87 75.64) (end 115.39 75.64) (width 0.25) (layer "F.Cu") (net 24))
 (segment (start 128.675 82.575) (end 128.945 82.845) (width 0.25) (layer "F.Cu") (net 24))
 (segment (start 115.39 75.64) (end 115.43 75.68) (width 0.25) (layer "F.Cu") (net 24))
 (segment (start 113.11 76.4) (end 113.87 75.64) (width 0.25) (layer "F.Cu") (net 24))
 (via (at 121.15 98.45) (size 0.8) (drill 0.4) (layers "F.Cu" "B.Cu") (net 24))
 (via (at 128.05 82.6) (size 0.8) (drill 0.4) (layers "F.Cu" "B.Cu") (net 24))
 (via (at 115.43 75.68) (size 0.8) (drill 0.4) (layers "F.Cu" "B.Cu") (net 24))
 (segment (start 118.676687 75.68) (end 125.596687 82.6) (width 0.25) (layer "B.Cu") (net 24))
 (segment (start 122.62 96.89) (end 125.85 96.89) (width 0.25) (layer "B.Cu") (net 24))
 (segment (start 115.43 75.68) (end 118.676687 75.68) (width 0.25) (layer "B.Cu") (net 24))
 (segment (start 121.06 98.45) (end 121.15 98.45) (width 0.25) (layer "B.Cu") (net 24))
 (segment (start 121.15 98.45) (end 121.15 98.36) (width 0.25) (layer "B.Cu") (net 24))
 (segment (start 121.15 98.36) (end 122.62 96.89) (width 0.25) (layer "B.Cu") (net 24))
 (segment (start 125.596687 82.6) (end 128.05 82.6) (width 0.25) (layer "B.Cu") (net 24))
 (segment (start 113.11 82.4) (end 115.36 82.4) (width 0.25) (layer "F.Cu") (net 23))
 (segment (start 125.85 94.35) (end 125.85 94.775305) (width 0.25) (layer "F.Cu") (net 23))
 (segment (start 112.71 82.4) (end 113.11 82.4) (width 0.25) (layer "F.Cu") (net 23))
 (via (at 115.36 82.4) (size 0.8) (drill 0.4) (layers "F.Cu" "B.Cu") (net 23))
 (segment (start 122.41 98.24) (end 118.7725 101.8775) (width 0.25) (layer "B.Cu") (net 23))
 (segment (start 115.36 82.4) (end 115.3 82.46) (width 0.25) (layer "B.Cu") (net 23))
 (segment (start 113.3475 96.0525) (end 118.24 91.16) (width 0.25) (layer "B.Cu") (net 23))
 (segment (start 115.42 82.46) (end 115.36 82.4) (width 0.25) (layer "B.Cu") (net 23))
 (segment (start 118.7725 101.8775) (end 113.999187 101.8775) (width 0.25) (layer "B.Cu") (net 23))
 (segment (start 118.24 84.48) (end 116.22 82.46) (width 0.25) (layer "B.Cu") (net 23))
 (segment (start 126.332914 98.24) (end 122.41 98.24) (width 0.25) (layer "B.Cu") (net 23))
 (segment (start 113.999187 101.8775) (end 113.3475 101.225813) (width 0.25) (layer "B.Cu") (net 23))
 (segment (start 118.24 91.16) (end 118.24 84.48) (width 0.25) (layer "B.Cu") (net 23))
 (segment (start 113.3475 101.225813) (end 113.3475 96.0525) (width 0.25) (layer "B.Cu") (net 23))
 (segment (start 125.85 94.35) (end 127.19 95.69) (width 0.25) (layer "B.Cu") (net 23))
 (segment (start 127.19 95.69) (end 127.19 97.382914) (width 0.25) (layer "B.Cu") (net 23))
 (segment (start 116.22 82.46) (end 115.42 82.46) (width 0.25) (layer "B.Cu") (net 23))
 (segment (start 127.19 97.382914) (end 126.332914 98.24) (width 0.25) (layer "B.Cu") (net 23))
 (segment (start 116.2975 80.77) (end 115.1025 79.575) (width 0.25) (layer "F.Cu") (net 1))
 (segment (start 81.96 84.74) (end 81.99 84.77) (width 0.25) (layer "F.Cu") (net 1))
 (segment (start 115.035 79.575) (end 114.98 79.63) (width 0.25) (layer "F.Cu") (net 1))
 (segment (start 81.99 84.71) (end 81.96 84.74) (width 0.25) (layer "F.Cu") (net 1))
 (segment (start 81.99 84.77) (end 81.99 88.46) (width 0.25) (layer "F.Cu") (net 1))
 (segment (start 114.98 79.63) (end 114.925 79.575) (width 0.25) (layer "F.Cu") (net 1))
 (segment (start 115.1025 79.575) (end 115.035 79.575) (width 0.25) (layer "F.Cu") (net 1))
 (segment (start 113.48 80.77) (end 113.11 80.4) (width 0.25) (layer "F.Cu") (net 1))
 (segment (start 116.2975 80.77) (end 113.48 80.77) (width 0.25) (layer "F.Cu") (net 1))
 (via (at 114.98 79.63) (size 0.8) (drill 0.4) (layers "F.Cu" "B.Cu") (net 1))
 (via (at 81.96 84.74) (size 0.8) (drill 0.4) (layers "F.Cu" "B.Cu") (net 1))
 (segment (start 114.06 80.55) (end 114.98 79.63) (width 0.25) (layer "B.Cu") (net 1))
 (segment (start 113.11 80.55) (end 114.06 80.55) (width 0.25) (layer "B.Cu") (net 1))
 (segment (start 83.4125 80.1425) (end 90.035 73.52) (width 0.25) (layer "B.Cu") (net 1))
 (segment (start 81.96 84.74) (end 83.4125 83.2875) (width 0.25) (layer "B.Cu") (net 1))
 (segment (start 90.035 73.52) (end 106.08 73.52) (width 0.25) (layer "B.Cu") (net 1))
 (segment (start 83.4125 83.2875) (end 83.4125 80.1425) (width 0.25) (layer "B.Cu") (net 1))
 (segment (start 106.08 73.52) (end 113.11 80.55) (width 0.25) (layer "B.Cu") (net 1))
 (segment (start 115.807076 78.99) (end 115.76 78.99) (width 0.25) (layer "F.Cu") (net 4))
 (segment (start 122.71 87.23) (end 122.68 87.2) (width 0.25) (layer "F.Cu") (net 4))
 (segment (start 124.51 86) (end 123.31 87.2) (width 0.25) (layer "F.Cu") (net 4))
 (segment (start 122.74 87.2) (end 122.71 87.23) (width 0.25) (layer "F.Cu") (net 4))
 (segment (start 115.305 78.4) (end 113.11 78.4) (width 0.25) (layer "F.Cu") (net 4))
 (segment (start 115.217076 78.4) (end 113.11 78.4) (width 0.25) (layer "F.Cu") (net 4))
 (segment (start 115.76 78.99) (end 115.76 78.942924) (width 0.25) (layer "F.Cu") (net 4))
 (segment (start 117.265 76.44) (end 115.305 78.4) (width 0.25) (layer "F.Cu") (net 4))
 (segment (start 123.31 87.2) (end 122.74 87.2) (width 0.25) (layer "F.Cu") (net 4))
 (segment (start 115.76 78.942924) (end 115.217076 78.4) (width 0.25) (layer "F.Cu") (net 4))
 (via (at 122.71 87.23) (size 0.8) (drill 0.4) (layers "F.Cu" "B.Cu") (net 4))
 (via (at 115.76 78.99) (size 0.8) (drill 0.4) (layers "F.Cu" "B.Cu") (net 4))
 (segment (start 119.79 79.01) (end 115.76 78.99) (width 0.25) (layer "B.Cu") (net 4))
 (segment (start 122.71 87.23) (end 119.79 79.01) (width 0.25) (layer "B.Cu") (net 4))
 (segment (start 95.1 78.4) (end 97.91 78.4) (width 0.25) (layer "F.Cu") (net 10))
 (segment (start 94.94 78.56) (end 95.1 78.4) (width 0.25) (layer "F.Cu") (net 10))
 (via (at 94.94 78.56) (size 0.8) (drill 0.4) (layers "F.Cu" "B.Cu") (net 10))
 (segment (start 90.9675 81.5025) (end 91.24 81.23) (width 0.25) (layer "B.Cu") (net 10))
 (segment (start 90.9675 89.69) (end 90.9675 81.5025) (width 0.25) (layer "B.Cu") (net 10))
 (segment (start 93.91 78.56) (end 94.94 78.56) (width 0.25) (layer "B.Cu") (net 10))
 (segment (start 91.24 81.23) (end 93.91 78.56) (width 0.25) (layer "B.Cu") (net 10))
 (segment (start 95.05 74.4) (end 97.91 74.4) (width 0.25) (layer "F.Cu") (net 8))
 (segment (start 94.94 74.29) (end 95.05 74.4) (width 0.25) (layer "F.Cu") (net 8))
 (via (at 94.94 74.29) (size 0.8) (drill 0.4) (layers "F.Cu" "B.Cu") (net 8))
 (segment (start 90.6575 93.74) (end 88.66 91.7425) (width 0.25) (layer "B.Cu") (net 8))
 (segment (start 91.3 74.29) (end 94.94 74.29) (width 0.25) (layer "B.Cu") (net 8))
 (segment (start 88.66 76.93) (end 90.77 74.82) (width 0.25) (layer "B.Cu") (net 8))
 (segment (start 88.66 83.87) (end 88.66 76.93) (width 0.25) (layer "B.Cu") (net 8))
 (segment (start 90.77 74.82) (end 91.3 74.29) (width 0.25) (layer "B.Cu") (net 8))
 (segment (start 88.66 91.7425) (end 88.66 83.87) (width 0.25) (layer "B.Cu") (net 8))
 (segment (start 116.6475 86.4) (end 113.11 86.4) (width 0.25) (layer "F.Cu") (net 7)))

